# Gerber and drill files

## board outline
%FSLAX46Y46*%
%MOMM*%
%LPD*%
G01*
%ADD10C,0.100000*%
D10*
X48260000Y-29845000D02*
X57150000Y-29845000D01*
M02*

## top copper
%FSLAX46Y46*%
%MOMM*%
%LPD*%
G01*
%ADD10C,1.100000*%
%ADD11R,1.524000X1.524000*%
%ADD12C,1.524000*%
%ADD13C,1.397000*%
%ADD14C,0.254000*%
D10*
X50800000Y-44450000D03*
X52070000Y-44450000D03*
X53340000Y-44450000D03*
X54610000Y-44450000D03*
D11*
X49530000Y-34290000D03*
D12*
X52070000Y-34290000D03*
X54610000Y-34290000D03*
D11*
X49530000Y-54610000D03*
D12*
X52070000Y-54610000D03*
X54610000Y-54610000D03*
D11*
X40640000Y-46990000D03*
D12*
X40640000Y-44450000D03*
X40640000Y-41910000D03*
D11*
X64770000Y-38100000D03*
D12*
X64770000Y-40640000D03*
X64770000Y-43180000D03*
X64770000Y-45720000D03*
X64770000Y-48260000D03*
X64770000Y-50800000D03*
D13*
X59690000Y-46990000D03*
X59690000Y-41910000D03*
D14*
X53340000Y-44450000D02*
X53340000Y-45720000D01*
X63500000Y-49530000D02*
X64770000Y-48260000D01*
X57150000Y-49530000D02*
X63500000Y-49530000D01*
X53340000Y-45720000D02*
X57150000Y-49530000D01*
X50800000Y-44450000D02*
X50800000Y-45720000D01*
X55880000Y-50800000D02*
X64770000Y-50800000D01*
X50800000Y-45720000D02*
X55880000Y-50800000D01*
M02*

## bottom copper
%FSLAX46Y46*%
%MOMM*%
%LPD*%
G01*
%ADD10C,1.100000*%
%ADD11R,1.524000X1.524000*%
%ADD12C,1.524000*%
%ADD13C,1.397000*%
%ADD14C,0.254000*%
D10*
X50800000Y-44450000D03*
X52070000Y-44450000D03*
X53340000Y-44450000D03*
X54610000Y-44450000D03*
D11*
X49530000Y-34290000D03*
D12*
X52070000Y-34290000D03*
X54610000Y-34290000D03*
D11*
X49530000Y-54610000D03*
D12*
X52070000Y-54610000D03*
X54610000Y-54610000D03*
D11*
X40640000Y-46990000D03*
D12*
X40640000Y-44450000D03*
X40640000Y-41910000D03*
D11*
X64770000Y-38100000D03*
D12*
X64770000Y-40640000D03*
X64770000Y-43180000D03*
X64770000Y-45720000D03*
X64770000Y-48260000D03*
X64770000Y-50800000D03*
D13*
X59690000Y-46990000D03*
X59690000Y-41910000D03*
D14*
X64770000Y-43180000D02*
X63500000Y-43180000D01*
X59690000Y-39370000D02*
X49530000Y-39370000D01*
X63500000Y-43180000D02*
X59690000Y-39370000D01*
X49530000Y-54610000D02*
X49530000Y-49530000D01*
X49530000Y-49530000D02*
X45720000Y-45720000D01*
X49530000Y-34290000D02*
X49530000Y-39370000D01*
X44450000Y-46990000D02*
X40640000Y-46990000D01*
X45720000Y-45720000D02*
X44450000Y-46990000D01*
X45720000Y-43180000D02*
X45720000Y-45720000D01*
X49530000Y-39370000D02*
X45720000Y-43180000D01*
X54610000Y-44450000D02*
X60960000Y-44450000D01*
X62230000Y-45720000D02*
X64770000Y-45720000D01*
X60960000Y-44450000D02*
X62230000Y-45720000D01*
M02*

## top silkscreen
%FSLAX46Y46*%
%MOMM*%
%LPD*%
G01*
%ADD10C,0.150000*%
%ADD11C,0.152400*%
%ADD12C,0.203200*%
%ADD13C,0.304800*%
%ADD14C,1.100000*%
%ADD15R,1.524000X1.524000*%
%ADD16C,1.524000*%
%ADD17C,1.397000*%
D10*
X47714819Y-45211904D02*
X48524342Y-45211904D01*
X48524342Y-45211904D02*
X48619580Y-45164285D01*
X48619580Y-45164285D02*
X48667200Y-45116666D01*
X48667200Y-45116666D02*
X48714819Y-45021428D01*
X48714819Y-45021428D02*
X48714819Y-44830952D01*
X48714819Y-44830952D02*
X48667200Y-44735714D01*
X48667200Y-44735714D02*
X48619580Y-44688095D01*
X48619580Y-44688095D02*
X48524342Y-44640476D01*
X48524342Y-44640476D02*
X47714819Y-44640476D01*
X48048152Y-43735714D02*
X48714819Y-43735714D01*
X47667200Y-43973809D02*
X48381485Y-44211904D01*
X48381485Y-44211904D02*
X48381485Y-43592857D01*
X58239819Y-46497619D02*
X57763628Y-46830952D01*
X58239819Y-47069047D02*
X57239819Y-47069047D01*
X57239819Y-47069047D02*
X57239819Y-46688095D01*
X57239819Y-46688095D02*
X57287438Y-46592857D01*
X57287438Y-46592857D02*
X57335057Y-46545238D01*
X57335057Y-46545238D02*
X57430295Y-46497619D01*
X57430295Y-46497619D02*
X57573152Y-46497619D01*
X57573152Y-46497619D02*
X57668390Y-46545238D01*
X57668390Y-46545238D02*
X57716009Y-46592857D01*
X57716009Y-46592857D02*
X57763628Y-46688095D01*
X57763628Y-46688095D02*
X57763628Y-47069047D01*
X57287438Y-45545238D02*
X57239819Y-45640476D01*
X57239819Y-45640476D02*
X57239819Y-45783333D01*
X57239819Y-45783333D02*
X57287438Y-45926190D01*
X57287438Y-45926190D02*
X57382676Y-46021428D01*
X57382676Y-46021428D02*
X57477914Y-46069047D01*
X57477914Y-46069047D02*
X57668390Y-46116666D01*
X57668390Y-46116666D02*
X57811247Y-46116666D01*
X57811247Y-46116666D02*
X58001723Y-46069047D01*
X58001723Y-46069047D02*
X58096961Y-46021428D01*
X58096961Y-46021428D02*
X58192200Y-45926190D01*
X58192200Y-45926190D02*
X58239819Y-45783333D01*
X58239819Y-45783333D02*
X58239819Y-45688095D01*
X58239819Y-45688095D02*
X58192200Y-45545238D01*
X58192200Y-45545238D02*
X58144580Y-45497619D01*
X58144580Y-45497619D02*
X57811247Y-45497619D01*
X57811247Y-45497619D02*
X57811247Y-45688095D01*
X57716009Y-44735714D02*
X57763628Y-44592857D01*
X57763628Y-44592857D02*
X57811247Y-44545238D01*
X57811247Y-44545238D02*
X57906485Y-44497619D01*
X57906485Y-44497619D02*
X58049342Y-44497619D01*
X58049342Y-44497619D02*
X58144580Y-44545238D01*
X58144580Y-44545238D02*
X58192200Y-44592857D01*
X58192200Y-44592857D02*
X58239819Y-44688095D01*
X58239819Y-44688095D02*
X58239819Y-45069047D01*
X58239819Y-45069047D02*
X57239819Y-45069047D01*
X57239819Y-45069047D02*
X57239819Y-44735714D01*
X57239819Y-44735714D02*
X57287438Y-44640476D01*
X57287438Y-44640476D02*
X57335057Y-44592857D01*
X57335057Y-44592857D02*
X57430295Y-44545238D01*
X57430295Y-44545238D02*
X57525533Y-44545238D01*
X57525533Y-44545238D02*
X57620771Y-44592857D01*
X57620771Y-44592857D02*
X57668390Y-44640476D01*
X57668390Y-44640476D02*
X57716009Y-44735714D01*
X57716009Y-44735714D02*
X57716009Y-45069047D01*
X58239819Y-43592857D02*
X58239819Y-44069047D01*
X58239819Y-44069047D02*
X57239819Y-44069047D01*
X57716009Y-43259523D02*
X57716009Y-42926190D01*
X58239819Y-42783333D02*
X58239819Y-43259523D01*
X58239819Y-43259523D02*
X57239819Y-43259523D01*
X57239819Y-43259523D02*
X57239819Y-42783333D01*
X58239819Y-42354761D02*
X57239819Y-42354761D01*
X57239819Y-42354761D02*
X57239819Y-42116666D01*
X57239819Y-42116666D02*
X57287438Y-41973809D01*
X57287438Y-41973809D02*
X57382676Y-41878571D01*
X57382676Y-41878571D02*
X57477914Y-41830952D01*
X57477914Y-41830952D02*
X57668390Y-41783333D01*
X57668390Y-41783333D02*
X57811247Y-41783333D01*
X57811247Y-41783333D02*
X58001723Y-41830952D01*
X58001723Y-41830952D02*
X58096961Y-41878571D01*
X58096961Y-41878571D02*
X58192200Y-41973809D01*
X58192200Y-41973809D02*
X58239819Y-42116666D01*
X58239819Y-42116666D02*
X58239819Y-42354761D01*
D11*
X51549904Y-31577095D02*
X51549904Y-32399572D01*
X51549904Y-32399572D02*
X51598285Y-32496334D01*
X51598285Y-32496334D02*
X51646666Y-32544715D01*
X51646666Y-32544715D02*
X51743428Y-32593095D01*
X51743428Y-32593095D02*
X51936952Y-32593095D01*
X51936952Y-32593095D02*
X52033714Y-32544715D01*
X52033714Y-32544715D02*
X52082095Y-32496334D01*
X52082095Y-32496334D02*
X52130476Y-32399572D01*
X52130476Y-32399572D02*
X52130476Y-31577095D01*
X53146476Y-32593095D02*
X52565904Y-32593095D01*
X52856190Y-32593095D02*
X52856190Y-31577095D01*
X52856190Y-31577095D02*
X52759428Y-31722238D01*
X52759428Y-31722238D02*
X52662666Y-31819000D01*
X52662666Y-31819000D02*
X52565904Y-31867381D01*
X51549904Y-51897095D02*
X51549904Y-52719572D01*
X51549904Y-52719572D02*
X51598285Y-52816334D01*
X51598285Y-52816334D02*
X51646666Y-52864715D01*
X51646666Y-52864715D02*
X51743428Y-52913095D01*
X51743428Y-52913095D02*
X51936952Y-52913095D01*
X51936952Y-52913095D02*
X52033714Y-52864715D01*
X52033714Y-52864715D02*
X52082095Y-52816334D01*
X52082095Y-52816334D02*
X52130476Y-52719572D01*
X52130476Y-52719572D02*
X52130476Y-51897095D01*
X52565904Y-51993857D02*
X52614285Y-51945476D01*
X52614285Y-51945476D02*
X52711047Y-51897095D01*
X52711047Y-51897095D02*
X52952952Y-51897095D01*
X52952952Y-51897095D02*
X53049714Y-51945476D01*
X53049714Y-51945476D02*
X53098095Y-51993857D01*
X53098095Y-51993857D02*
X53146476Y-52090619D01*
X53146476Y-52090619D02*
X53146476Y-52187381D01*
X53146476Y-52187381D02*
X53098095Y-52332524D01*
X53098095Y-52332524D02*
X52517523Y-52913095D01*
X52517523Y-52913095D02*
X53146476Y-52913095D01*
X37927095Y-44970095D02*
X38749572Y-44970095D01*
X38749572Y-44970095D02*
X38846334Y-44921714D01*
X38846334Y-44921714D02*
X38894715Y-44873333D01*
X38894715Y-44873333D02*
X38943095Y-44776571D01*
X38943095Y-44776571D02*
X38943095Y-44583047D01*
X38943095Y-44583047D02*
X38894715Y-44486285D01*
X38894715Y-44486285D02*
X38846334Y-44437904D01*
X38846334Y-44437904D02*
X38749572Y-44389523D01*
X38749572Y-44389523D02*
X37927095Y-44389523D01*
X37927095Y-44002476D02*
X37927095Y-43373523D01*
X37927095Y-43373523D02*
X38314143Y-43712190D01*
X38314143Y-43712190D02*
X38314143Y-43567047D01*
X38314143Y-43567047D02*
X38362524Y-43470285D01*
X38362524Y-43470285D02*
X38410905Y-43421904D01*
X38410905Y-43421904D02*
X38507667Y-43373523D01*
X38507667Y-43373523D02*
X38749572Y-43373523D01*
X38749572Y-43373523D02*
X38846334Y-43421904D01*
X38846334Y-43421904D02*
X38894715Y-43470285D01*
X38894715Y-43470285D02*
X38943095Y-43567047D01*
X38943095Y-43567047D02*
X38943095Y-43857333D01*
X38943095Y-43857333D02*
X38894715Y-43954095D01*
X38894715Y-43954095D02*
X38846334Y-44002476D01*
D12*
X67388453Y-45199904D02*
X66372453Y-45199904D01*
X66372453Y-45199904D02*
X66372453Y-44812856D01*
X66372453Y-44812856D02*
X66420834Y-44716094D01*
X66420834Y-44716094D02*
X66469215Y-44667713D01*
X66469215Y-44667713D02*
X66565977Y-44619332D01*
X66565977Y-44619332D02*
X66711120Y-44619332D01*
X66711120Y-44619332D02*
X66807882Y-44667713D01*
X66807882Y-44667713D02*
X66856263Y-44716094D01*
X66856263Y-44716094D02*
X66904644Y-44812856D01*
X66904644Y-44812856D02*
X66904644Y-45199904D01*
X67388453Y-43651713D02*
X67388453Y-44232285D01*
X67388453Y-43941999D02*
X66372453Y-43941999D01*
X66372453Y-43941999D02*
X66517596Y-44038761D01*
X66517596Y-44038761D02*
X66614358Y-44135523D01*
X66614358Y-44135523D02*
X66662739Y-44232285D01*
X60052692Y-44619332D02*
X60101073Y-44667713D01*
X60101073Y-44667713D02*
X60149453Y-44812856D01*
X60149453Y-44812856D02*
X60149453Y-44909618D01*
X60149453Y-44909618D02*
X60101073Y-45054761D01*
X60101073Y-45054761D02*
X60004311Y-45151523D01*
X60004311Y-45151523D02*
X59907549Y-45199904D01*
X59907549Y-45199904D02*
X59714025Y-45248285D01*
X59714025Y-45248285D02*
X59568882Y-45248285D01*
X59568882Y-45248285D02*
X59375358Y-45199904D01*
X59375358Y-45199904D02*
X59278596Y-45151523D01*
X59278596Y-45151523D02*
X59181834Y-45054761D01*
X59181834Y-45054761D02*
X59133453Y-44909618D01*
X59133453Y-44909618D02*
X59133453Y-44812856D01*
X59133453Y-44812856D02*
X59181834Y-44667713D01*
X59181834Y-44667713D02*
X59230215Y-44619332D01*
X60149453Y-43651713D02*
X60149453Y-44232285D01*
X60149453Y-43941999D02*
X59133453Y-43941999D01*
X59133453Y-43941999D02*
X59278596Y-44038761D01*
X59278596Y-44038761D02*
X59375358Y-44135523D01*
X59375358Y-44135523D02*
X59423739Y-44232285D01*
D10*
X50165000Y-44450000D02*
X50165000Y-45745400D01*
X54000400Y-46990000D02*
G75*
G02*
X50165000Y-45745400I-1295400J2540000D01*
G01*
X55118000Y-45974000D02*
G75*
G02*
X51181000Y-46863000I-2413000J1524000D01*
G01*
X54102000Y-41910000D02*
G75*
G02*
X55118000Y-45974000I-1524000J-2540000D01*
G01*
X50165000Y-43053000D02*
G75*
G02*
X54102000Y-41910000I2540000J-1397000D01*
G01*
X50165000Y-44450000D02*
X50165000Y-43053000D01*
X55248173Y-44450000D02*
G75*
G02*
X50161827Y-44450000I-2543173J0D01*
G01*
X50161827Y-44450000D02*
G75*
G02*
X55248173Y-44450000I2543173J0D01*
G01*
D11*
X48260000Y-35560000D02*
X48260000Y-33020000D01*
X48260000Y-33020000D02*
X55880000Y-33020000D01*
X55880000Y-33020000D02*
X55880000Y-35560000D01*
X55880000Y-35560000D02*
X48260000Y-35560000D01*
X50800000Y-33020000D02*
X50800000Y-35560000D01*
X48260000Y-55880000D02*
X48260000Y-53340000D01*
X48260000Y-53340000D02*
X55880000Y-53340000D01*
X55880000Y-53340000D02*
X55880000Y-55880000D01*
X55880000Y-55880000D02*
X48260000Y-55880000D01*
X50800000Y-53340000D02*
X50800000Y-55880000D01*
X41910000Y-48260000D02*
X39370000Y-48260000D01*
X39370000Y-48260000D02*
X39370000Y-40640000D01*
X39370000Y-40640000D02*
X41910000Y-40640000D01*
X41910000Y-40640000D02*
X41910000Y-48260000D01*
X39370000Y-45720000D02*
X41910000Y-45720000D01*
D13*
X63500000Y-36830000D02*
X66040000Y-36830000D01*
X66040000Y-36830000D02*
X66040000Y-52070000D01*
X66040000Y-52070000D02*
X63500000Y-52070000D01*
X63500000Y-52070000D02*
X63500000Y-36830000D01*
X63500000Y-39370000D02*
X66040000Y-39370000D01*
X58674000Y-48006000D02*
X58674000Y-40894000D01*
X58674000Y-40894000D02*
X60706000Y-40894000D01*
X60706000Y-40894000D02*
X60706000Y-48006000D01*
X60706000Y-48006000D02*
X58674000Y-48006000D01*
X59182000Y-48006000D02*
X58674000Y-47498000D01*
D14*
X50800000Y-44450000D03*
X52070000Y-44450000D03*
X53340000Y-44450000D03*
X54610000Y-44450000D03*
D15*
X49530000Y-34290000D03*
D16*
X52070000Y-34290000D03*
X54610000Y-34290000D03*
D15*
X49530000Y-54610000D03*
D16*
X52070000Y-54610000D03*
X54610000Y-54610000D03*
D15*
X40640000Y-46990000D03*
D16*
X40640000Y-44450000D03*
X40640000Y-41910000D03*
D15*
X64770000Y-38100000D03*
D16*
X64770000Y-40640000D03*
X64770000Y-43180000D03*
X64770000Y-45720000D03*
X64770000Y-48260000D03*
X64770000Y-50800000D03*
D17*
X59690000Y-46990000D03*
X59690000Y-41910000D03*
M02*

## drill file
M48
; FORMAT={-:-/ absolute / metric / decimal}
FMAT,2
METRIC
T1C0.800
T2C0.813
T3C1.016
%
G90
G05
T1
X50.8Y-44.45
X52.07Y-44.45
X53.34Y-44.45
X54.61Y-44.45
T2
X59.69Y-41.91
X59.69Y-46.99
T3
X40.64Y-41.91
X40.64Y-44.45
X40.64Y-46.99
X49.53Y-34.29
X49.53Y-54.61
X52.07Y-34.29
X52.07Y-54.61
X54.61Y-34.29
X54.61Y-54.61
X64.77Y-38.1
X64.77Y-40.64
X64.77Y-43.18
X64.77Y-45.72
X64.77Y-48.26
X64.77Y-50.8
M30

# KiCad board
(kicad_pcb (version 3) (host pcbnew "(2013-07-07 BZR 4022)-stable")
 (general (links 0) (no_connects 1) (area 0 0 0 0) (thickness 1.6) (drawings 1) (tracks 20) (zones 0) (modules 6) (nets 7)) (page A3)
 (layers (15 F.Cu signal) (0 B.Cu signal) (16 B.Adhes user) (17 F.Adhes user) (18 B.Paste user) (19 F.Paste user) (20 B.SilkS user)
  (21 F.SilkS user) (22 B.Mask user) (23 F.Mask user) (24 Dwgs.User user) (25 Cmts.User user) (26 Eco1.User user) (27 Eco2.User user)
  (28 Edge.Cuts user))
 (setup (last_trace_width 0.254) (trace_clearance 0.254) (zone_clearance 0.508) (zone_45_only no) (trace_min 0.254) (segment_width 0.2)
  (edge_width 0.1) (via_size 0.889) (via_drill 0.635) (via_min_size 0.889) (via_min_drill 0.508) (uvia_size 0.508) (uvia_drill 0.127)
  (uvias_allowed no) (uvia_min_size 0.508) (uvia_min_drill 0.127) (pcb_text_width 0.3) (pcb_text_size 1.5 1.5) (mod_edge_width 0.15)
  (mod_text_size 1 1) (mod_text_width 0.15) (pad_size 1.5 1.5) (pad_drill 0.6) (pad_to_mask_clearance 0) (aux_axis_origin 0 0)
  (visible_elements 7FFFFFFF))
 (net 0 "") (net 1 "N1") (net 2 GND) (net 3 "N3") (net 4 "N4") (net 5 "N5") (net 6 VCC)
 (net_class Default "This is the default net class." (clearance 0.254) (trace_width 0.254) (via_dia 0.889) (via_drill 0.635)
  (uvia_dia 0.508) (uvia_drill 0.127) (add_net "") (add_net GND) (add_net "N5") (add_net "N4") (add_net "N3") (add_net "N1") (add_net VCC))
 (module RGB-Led (layer F.Cu) (at 53.34 44.45 90)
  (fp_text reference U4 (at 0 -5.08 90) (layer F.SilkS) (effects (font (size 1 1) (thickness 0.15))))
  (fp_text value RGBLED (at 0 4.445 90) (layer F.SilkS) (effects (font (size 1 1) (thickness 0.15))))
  (fp_line (start 0 -3.175) (end -1.2954 -3.175) (layer F.SilkS) (width 0.15))
  (fp_arc (start 0 -0.635) (end -2.54 0.6604) (angle 90) (layer F.SilkS) (width 0.15))
  (fp_arc (start 0 -0.635) (end -1.524 1.778) (angle 90) (layer F.SilkS) (width 0.15))
  (fp_arc (start 0 -0.762) (end 2.54 0.762) (angle 90) (layer F.SilkS) (width 0.15))
  (fp_arc (start 0 -0.635) (end 1.397 -3.175) (angle 90) (layer F.SilkS) (width 0.15))
  (fp_line (start 0 -3.175) (end 1.397 -3.175) (layer F.SilkS) (width 0.15))
  (fp_circle (center 0 -0.635) (end 2.54 -0.508) (layer F.SilkS) (width 0.15))
  (pad 1 thru_hole circle (at 0 -2.54 90) (size 1.1 1.1) (drill 0.8) (layers *.Cu *.Mask F.SilkS) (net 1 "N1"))
  (pad 2 thru_hole circle (at 0 -1.27 90) (size 1.1 1.1) (drill 0.8) (layers *.Cu *.Mask F.SilkS) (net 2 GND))
  (pad 3 thru_hole circle (at 0 0 90) (size 1.1 1.1) (drill 0.8) (layers *.Cu *.Mask F.SilkS) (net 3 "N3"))
  (pad 4 thru_hole circle (at 0 1.27 90) (size 1.1 1.1) (drill 0.8) (layers *.Cu *.Mask F.SilkS) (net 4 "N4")))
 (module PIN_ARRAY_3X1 (layer F.Cu) (at 52.07 34.29)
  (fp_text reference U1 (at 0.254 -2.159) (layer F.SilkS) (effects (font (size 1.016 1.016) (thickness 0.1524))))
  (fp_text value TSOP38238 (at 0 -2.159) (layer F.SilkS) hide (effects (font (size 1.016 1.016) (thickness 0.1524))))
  (fp_line (start -3.81 1.27) (end -3.81 -1.27) (layer F.SilkS) (width 0.1524))
  (fp_line (start -3.81 -1.27) (end 3.81 -1.27) (layer F.SilkS) (width 0.1524))
  (fp_line (start 3.81 -1.27) (end 3.81 1.27) (layer F.SilkS) (width 0.1524))
  (fp_line (start 3.81 1.27) (end -3.81 1.27) (layer F.SilkS) (width 0.1524))
  (fp_line (start -1.27 -1.27) (end -1.27 1.27) (layer F.SilkS) (width 0.1524))
  (pad 1 thru_hole rect (at -2.54 0) (size 1.524 1.524) (drill 1.016) (layers *.Cu *.Mask F.SilkS) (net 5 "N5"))
  (pad 2 thru_hole circle (at 0 0) (size 1.524 1.524) (drill 1.016) (layers *.Cu *.Mask F.SilkS) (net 2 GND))
  (pad 3 thru_hole circle (at 2.54 0) (size 1.524 1.524) (drill 1.016) (layers *.Cu *.Mask F.SilkS) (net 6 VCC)))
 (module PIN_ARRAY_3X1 (layer F.Cu) (at 52.07 54.61)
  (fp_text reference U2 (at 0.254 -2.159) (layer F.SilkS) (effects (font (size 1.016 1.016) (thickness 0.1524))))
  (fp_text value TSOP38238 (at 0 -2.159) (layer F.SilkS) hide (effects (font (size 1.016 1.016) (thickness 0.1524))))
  (fp_line (start -3.81 1.27) (end -3.81 -1.27) (layer F.SilkS) (width 0.1524))
  (fp_line (start -3.81 -1.27) (end 3.81 -1.27) (layer F.SilkS) (width 0.1524))
  (fp_line (start 3.81 -1.27) (end 3.81 1.27) (layer F.SilkS) (width 0.1524))
  (fp_line (start 3.81 1.27) (end -3.81 1.27) (layer F.SilkS) (width 0.1524))
  (fp_line (start -1.27 -1.27) (end -1.27 1.27) (layer F.SilkS) (width 0.1524))
  (pad 1 thru_hole rect (at -2.54 0) (size 1.524 1.524) (drill 1.016) (layers *.Cu *.Mask F.SilkS) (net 5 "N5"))
  (pad 2 thru_hole circle (at 0 0) (size 1.524 1.524) (drill 1.016) (layers *.Cu *.Mask F.SilkS) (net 2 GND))
  (pad 3 thru_hole circle (at 2.54 0) (size 1.524 1.524) (drill 1.016) (layers *.Cu *.Mask F.SilkS) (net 6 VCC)))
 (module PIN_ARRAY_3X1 (layer F.Cu) (at 40.64 44.45 90)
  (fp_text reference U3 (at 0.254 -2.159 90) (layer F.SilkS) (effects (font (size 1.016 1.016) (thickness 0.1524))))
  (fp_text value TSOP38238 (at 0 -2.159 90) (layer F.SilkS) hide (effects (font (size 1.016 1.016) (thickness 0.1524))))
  (fp_line (start -3.81 1.27) (end -3.81 -1.27) (layer F.SilkS) (width 0.1524))
  (fp_line (start -3.81 -1.27) (end 3.81 -1.27) (layer F.SilkS) (width 0.1524))
  (fp_line (start 3.81 -1.27) (end 3.81 1.27) (layer F.SilkS) (width 0.1524))
  (fp_line (start 3.81 1.27) (end -3.81 1.27) (layer F.SilkS) (width 0.1524))
  (fp_line (start -1.27 -1.27) (end -1.27 1.27) (layer F.SilkS) (width 0.1524))
  (pad 1 thru_hole rect (at -2.54 0 90) (size 1.524 1.524) (drill 1.016) (layers *.Cu *.Mask F.SilkS) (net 5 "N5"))
  (pad 2 thru_hole circle (at 0 0 90) (size 1.524 1.524) (drill 1.016) (layers *.Cu *.Mask F.SilkS) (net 2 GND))
  (pad 3 thru_hole circle (at 2.54 0 90) (size 1.524 1.524) (drill 1.016) (layers *.Cu *.Mask F.SilkS) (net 6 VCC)))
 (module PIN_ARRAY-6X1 (layer F.Cu) (at 64.77 44.45 270)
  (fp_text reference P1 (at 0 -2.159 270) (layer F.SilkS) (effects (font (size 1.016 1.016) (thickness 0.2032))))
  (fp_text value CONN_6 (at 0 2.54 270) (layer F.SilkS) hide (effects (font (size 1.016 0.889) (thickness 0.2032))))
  (fp_line (start -7.62 1.27) (end -7.62 -1.27) (layer F.SilkS) (width 0.3048))
  (fp_line (start -7.62 -1.27) (end 7.62 -1.27) (layer F.SilkS) (width 0.3048))
  (fp_line (start 7.62 -1.27) (end 7.62 1.27) (layer F.SilkS) (width 0.3048))
  (fp_line (start 7.62 1.27) (end -7.62 1.27) (layer F.SilkS) (width 0.3048))
  (fp_line (start -5.08 1.27) (end -5.08 -1.27) (layer F.SilkS) (width 0.3048))
  (pad 1 thru_hole rect (at -6.35 0 270) (size 1.524 1.524) (drill 1.016) (layers *.Cu *.Mask F.SilkS) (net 2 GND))
  (pad 2 thru_hole circle (at -3.81 0 270) (size 1.524 1.524) (drill 1.016) (layers *.Cu *.Mask F.SilkS) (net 6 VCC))
  (pad 3 thru_hole circle (at -1.27 0 270) (size 1.524 1.524) (drill 1.016) (layers *.Cu *.Mask F.SilkS) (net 5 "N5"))
  (pad 4 thru_hole circle (at 1.27 0 270) (size 1.524 1.524) (drill 1.016) (layers *.Cu *.Mask F.SilkS) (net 4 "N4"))
  (pad 5 thru_hole circle (at 3.81 0 270) (size 1.524 1.524) (drill 1.016) (layers *.Cu *.Mask F.SilkS) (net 3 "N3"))
  (pad 6 thru_hole circle (at 6.35 0 270) (size 1.524 1.524) (drill 1.016) (layers *.Cu *.Mask F.SilkS) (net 1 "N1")))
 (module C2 (layer F.Cu) (at 59.69 44.45 90)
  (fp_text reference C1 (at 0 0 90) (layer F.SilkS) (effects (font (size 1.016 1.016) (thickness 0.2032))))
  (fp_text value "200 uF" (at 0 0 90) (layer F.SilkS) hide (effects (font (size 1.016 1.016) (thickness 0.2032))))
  (fp_line (start -3.556 -1.016) (end 3.556 -1.016) (layer F.SilkS) (width 0.3048))
  (fp_line (start 3.556 -1.016) (end 3.556 1.016) (layer F.SilkS) (width 0.3048))
  (fp_line (start 3.556 1.016) (end -3.556 1.016) (layer F.SilkS) (width 0.3048))
  (fp_line (start -3.556 1.016) (end -3.556 -1.016) (layer F.SilkS) (width 0.3048))
  (fp_line (start -3.556 -0.508) (end -3.048 -1.016) (layer F.SilkS) (width 0.3048))
  (pad 1 thru_hole circle (at -2.54 0 90) (size 1.397 1.397) (drill 0.8128) (layers *.Cu *.Mask F.SilkS) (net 6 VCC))
  (pad 2 thru_hole circle (at 2.54 0 90) (size 1.397 1.397) (drill 0.8128) (layers *.Cu *.Mask F.SilkS) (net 2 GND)))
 (gr_line (start 48.26 29.845) (end 57.15 29.845) (angle 90) (layer Edge.Cuts) (width 0.1))
 (segment (start 64.77 43.18) (end 63.5 43.18) (width 0.254) (layer B.Cu) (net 5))
 (segment (start 59.69 39.37) (end 49.53 39.37) (width 0.254) (layer B.Cu) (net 5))
 (segment (start 63.5 43.18) (end 59.69 39.37) (width 0.254) (layer B.Cu) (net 5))
 (segment (start 49.53 54.61) (end 49.53 49.53) (width 0.254) (layer B.Cu) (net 5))
 (segment (start 49.53 49.53) (end 45.72 45.72) (width 0.254) (layer B.Cu) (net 5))
 (segment (start 49.53 34.29) (end 49.53 39.37) (width 0.254) (layer B.Cu) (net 5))
 (segment (start 44.45 46.99) (end 40.64 46.99) (width 0.254) (layer B.Cu) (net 5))
 (segment (start 45.72 45.72) (end 44.45 46.99) (width 0.254) (layer B.Cu) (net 5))
 (segment (start 45.72 43.18) (end 45.72 45.72) (width 0.254) (layer B.Cu) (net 5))
 (segment (start 49.53 39.37) (end 45.72 43.18) (width 0.254) (layer B.Cu) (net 5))
 (segment (start 54.61 44.45) (end 60.96 44.45) (width 0.254) (layer B.Cu) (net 4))
 (segment (start 62.23 45.72) (end 64.77 45.72) (width 0.254) (layer B.Cu) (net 4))
 (segment (start 60.96 44.45) (end 62.23 45.72) (width 0.254) (layer B.Cu) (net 4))
 (segment (start 53.34 44.45) (end 53.34 45.72) (width 0.254) (layer F.Cu) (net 3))
 (segment (start 63.5 49.53) (end 64.77 48.26) (width 0.254) (layer F.Cu) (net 3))
 (segment (start 57.15 49.53) (end 63.5 49.53) (width 0.254) (layer F.Cu) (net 3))
 (segment (start 53.34 45.72) (end 57.15 49.53) (width 0.254) (layer F.Cu) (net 3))
 (segment (start 50.8 44.45) (end 50.8 45.72) (width 0.254) (layer F.Cu) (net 1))
 (segment (start 55.88 50.8) (end 64.77 50.8) (width 0.254) (layer F.Cu) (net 1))
 (segment (start 50.8 45.72) (end 55.88 50.8) (width 0.254) (layer F.Cu) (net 1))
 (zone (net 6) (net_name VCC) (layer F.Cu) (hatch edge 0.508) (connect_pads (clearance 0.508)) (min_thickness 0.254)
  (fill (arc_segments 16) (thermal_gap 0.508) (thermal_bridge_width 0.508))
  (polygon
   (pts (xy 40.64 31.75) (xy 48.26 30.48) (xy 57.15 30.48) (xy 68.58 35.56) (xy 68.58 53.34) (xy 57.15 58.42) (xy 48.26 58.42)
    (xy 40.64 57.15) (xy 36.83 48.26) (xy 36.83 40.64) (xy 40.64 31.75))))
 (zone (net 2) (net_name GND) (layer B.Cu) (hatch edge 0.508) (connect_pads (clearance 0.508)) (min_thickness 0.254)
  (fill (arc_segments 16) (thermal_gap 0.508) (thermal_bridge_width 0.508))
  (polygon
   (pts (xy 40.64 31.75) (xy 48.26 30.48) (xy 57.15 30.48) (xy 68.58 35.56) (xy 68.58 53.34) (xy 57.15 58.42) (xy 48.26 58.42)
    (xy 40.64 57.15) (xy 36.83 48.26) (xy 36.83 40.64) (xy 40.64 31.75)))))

